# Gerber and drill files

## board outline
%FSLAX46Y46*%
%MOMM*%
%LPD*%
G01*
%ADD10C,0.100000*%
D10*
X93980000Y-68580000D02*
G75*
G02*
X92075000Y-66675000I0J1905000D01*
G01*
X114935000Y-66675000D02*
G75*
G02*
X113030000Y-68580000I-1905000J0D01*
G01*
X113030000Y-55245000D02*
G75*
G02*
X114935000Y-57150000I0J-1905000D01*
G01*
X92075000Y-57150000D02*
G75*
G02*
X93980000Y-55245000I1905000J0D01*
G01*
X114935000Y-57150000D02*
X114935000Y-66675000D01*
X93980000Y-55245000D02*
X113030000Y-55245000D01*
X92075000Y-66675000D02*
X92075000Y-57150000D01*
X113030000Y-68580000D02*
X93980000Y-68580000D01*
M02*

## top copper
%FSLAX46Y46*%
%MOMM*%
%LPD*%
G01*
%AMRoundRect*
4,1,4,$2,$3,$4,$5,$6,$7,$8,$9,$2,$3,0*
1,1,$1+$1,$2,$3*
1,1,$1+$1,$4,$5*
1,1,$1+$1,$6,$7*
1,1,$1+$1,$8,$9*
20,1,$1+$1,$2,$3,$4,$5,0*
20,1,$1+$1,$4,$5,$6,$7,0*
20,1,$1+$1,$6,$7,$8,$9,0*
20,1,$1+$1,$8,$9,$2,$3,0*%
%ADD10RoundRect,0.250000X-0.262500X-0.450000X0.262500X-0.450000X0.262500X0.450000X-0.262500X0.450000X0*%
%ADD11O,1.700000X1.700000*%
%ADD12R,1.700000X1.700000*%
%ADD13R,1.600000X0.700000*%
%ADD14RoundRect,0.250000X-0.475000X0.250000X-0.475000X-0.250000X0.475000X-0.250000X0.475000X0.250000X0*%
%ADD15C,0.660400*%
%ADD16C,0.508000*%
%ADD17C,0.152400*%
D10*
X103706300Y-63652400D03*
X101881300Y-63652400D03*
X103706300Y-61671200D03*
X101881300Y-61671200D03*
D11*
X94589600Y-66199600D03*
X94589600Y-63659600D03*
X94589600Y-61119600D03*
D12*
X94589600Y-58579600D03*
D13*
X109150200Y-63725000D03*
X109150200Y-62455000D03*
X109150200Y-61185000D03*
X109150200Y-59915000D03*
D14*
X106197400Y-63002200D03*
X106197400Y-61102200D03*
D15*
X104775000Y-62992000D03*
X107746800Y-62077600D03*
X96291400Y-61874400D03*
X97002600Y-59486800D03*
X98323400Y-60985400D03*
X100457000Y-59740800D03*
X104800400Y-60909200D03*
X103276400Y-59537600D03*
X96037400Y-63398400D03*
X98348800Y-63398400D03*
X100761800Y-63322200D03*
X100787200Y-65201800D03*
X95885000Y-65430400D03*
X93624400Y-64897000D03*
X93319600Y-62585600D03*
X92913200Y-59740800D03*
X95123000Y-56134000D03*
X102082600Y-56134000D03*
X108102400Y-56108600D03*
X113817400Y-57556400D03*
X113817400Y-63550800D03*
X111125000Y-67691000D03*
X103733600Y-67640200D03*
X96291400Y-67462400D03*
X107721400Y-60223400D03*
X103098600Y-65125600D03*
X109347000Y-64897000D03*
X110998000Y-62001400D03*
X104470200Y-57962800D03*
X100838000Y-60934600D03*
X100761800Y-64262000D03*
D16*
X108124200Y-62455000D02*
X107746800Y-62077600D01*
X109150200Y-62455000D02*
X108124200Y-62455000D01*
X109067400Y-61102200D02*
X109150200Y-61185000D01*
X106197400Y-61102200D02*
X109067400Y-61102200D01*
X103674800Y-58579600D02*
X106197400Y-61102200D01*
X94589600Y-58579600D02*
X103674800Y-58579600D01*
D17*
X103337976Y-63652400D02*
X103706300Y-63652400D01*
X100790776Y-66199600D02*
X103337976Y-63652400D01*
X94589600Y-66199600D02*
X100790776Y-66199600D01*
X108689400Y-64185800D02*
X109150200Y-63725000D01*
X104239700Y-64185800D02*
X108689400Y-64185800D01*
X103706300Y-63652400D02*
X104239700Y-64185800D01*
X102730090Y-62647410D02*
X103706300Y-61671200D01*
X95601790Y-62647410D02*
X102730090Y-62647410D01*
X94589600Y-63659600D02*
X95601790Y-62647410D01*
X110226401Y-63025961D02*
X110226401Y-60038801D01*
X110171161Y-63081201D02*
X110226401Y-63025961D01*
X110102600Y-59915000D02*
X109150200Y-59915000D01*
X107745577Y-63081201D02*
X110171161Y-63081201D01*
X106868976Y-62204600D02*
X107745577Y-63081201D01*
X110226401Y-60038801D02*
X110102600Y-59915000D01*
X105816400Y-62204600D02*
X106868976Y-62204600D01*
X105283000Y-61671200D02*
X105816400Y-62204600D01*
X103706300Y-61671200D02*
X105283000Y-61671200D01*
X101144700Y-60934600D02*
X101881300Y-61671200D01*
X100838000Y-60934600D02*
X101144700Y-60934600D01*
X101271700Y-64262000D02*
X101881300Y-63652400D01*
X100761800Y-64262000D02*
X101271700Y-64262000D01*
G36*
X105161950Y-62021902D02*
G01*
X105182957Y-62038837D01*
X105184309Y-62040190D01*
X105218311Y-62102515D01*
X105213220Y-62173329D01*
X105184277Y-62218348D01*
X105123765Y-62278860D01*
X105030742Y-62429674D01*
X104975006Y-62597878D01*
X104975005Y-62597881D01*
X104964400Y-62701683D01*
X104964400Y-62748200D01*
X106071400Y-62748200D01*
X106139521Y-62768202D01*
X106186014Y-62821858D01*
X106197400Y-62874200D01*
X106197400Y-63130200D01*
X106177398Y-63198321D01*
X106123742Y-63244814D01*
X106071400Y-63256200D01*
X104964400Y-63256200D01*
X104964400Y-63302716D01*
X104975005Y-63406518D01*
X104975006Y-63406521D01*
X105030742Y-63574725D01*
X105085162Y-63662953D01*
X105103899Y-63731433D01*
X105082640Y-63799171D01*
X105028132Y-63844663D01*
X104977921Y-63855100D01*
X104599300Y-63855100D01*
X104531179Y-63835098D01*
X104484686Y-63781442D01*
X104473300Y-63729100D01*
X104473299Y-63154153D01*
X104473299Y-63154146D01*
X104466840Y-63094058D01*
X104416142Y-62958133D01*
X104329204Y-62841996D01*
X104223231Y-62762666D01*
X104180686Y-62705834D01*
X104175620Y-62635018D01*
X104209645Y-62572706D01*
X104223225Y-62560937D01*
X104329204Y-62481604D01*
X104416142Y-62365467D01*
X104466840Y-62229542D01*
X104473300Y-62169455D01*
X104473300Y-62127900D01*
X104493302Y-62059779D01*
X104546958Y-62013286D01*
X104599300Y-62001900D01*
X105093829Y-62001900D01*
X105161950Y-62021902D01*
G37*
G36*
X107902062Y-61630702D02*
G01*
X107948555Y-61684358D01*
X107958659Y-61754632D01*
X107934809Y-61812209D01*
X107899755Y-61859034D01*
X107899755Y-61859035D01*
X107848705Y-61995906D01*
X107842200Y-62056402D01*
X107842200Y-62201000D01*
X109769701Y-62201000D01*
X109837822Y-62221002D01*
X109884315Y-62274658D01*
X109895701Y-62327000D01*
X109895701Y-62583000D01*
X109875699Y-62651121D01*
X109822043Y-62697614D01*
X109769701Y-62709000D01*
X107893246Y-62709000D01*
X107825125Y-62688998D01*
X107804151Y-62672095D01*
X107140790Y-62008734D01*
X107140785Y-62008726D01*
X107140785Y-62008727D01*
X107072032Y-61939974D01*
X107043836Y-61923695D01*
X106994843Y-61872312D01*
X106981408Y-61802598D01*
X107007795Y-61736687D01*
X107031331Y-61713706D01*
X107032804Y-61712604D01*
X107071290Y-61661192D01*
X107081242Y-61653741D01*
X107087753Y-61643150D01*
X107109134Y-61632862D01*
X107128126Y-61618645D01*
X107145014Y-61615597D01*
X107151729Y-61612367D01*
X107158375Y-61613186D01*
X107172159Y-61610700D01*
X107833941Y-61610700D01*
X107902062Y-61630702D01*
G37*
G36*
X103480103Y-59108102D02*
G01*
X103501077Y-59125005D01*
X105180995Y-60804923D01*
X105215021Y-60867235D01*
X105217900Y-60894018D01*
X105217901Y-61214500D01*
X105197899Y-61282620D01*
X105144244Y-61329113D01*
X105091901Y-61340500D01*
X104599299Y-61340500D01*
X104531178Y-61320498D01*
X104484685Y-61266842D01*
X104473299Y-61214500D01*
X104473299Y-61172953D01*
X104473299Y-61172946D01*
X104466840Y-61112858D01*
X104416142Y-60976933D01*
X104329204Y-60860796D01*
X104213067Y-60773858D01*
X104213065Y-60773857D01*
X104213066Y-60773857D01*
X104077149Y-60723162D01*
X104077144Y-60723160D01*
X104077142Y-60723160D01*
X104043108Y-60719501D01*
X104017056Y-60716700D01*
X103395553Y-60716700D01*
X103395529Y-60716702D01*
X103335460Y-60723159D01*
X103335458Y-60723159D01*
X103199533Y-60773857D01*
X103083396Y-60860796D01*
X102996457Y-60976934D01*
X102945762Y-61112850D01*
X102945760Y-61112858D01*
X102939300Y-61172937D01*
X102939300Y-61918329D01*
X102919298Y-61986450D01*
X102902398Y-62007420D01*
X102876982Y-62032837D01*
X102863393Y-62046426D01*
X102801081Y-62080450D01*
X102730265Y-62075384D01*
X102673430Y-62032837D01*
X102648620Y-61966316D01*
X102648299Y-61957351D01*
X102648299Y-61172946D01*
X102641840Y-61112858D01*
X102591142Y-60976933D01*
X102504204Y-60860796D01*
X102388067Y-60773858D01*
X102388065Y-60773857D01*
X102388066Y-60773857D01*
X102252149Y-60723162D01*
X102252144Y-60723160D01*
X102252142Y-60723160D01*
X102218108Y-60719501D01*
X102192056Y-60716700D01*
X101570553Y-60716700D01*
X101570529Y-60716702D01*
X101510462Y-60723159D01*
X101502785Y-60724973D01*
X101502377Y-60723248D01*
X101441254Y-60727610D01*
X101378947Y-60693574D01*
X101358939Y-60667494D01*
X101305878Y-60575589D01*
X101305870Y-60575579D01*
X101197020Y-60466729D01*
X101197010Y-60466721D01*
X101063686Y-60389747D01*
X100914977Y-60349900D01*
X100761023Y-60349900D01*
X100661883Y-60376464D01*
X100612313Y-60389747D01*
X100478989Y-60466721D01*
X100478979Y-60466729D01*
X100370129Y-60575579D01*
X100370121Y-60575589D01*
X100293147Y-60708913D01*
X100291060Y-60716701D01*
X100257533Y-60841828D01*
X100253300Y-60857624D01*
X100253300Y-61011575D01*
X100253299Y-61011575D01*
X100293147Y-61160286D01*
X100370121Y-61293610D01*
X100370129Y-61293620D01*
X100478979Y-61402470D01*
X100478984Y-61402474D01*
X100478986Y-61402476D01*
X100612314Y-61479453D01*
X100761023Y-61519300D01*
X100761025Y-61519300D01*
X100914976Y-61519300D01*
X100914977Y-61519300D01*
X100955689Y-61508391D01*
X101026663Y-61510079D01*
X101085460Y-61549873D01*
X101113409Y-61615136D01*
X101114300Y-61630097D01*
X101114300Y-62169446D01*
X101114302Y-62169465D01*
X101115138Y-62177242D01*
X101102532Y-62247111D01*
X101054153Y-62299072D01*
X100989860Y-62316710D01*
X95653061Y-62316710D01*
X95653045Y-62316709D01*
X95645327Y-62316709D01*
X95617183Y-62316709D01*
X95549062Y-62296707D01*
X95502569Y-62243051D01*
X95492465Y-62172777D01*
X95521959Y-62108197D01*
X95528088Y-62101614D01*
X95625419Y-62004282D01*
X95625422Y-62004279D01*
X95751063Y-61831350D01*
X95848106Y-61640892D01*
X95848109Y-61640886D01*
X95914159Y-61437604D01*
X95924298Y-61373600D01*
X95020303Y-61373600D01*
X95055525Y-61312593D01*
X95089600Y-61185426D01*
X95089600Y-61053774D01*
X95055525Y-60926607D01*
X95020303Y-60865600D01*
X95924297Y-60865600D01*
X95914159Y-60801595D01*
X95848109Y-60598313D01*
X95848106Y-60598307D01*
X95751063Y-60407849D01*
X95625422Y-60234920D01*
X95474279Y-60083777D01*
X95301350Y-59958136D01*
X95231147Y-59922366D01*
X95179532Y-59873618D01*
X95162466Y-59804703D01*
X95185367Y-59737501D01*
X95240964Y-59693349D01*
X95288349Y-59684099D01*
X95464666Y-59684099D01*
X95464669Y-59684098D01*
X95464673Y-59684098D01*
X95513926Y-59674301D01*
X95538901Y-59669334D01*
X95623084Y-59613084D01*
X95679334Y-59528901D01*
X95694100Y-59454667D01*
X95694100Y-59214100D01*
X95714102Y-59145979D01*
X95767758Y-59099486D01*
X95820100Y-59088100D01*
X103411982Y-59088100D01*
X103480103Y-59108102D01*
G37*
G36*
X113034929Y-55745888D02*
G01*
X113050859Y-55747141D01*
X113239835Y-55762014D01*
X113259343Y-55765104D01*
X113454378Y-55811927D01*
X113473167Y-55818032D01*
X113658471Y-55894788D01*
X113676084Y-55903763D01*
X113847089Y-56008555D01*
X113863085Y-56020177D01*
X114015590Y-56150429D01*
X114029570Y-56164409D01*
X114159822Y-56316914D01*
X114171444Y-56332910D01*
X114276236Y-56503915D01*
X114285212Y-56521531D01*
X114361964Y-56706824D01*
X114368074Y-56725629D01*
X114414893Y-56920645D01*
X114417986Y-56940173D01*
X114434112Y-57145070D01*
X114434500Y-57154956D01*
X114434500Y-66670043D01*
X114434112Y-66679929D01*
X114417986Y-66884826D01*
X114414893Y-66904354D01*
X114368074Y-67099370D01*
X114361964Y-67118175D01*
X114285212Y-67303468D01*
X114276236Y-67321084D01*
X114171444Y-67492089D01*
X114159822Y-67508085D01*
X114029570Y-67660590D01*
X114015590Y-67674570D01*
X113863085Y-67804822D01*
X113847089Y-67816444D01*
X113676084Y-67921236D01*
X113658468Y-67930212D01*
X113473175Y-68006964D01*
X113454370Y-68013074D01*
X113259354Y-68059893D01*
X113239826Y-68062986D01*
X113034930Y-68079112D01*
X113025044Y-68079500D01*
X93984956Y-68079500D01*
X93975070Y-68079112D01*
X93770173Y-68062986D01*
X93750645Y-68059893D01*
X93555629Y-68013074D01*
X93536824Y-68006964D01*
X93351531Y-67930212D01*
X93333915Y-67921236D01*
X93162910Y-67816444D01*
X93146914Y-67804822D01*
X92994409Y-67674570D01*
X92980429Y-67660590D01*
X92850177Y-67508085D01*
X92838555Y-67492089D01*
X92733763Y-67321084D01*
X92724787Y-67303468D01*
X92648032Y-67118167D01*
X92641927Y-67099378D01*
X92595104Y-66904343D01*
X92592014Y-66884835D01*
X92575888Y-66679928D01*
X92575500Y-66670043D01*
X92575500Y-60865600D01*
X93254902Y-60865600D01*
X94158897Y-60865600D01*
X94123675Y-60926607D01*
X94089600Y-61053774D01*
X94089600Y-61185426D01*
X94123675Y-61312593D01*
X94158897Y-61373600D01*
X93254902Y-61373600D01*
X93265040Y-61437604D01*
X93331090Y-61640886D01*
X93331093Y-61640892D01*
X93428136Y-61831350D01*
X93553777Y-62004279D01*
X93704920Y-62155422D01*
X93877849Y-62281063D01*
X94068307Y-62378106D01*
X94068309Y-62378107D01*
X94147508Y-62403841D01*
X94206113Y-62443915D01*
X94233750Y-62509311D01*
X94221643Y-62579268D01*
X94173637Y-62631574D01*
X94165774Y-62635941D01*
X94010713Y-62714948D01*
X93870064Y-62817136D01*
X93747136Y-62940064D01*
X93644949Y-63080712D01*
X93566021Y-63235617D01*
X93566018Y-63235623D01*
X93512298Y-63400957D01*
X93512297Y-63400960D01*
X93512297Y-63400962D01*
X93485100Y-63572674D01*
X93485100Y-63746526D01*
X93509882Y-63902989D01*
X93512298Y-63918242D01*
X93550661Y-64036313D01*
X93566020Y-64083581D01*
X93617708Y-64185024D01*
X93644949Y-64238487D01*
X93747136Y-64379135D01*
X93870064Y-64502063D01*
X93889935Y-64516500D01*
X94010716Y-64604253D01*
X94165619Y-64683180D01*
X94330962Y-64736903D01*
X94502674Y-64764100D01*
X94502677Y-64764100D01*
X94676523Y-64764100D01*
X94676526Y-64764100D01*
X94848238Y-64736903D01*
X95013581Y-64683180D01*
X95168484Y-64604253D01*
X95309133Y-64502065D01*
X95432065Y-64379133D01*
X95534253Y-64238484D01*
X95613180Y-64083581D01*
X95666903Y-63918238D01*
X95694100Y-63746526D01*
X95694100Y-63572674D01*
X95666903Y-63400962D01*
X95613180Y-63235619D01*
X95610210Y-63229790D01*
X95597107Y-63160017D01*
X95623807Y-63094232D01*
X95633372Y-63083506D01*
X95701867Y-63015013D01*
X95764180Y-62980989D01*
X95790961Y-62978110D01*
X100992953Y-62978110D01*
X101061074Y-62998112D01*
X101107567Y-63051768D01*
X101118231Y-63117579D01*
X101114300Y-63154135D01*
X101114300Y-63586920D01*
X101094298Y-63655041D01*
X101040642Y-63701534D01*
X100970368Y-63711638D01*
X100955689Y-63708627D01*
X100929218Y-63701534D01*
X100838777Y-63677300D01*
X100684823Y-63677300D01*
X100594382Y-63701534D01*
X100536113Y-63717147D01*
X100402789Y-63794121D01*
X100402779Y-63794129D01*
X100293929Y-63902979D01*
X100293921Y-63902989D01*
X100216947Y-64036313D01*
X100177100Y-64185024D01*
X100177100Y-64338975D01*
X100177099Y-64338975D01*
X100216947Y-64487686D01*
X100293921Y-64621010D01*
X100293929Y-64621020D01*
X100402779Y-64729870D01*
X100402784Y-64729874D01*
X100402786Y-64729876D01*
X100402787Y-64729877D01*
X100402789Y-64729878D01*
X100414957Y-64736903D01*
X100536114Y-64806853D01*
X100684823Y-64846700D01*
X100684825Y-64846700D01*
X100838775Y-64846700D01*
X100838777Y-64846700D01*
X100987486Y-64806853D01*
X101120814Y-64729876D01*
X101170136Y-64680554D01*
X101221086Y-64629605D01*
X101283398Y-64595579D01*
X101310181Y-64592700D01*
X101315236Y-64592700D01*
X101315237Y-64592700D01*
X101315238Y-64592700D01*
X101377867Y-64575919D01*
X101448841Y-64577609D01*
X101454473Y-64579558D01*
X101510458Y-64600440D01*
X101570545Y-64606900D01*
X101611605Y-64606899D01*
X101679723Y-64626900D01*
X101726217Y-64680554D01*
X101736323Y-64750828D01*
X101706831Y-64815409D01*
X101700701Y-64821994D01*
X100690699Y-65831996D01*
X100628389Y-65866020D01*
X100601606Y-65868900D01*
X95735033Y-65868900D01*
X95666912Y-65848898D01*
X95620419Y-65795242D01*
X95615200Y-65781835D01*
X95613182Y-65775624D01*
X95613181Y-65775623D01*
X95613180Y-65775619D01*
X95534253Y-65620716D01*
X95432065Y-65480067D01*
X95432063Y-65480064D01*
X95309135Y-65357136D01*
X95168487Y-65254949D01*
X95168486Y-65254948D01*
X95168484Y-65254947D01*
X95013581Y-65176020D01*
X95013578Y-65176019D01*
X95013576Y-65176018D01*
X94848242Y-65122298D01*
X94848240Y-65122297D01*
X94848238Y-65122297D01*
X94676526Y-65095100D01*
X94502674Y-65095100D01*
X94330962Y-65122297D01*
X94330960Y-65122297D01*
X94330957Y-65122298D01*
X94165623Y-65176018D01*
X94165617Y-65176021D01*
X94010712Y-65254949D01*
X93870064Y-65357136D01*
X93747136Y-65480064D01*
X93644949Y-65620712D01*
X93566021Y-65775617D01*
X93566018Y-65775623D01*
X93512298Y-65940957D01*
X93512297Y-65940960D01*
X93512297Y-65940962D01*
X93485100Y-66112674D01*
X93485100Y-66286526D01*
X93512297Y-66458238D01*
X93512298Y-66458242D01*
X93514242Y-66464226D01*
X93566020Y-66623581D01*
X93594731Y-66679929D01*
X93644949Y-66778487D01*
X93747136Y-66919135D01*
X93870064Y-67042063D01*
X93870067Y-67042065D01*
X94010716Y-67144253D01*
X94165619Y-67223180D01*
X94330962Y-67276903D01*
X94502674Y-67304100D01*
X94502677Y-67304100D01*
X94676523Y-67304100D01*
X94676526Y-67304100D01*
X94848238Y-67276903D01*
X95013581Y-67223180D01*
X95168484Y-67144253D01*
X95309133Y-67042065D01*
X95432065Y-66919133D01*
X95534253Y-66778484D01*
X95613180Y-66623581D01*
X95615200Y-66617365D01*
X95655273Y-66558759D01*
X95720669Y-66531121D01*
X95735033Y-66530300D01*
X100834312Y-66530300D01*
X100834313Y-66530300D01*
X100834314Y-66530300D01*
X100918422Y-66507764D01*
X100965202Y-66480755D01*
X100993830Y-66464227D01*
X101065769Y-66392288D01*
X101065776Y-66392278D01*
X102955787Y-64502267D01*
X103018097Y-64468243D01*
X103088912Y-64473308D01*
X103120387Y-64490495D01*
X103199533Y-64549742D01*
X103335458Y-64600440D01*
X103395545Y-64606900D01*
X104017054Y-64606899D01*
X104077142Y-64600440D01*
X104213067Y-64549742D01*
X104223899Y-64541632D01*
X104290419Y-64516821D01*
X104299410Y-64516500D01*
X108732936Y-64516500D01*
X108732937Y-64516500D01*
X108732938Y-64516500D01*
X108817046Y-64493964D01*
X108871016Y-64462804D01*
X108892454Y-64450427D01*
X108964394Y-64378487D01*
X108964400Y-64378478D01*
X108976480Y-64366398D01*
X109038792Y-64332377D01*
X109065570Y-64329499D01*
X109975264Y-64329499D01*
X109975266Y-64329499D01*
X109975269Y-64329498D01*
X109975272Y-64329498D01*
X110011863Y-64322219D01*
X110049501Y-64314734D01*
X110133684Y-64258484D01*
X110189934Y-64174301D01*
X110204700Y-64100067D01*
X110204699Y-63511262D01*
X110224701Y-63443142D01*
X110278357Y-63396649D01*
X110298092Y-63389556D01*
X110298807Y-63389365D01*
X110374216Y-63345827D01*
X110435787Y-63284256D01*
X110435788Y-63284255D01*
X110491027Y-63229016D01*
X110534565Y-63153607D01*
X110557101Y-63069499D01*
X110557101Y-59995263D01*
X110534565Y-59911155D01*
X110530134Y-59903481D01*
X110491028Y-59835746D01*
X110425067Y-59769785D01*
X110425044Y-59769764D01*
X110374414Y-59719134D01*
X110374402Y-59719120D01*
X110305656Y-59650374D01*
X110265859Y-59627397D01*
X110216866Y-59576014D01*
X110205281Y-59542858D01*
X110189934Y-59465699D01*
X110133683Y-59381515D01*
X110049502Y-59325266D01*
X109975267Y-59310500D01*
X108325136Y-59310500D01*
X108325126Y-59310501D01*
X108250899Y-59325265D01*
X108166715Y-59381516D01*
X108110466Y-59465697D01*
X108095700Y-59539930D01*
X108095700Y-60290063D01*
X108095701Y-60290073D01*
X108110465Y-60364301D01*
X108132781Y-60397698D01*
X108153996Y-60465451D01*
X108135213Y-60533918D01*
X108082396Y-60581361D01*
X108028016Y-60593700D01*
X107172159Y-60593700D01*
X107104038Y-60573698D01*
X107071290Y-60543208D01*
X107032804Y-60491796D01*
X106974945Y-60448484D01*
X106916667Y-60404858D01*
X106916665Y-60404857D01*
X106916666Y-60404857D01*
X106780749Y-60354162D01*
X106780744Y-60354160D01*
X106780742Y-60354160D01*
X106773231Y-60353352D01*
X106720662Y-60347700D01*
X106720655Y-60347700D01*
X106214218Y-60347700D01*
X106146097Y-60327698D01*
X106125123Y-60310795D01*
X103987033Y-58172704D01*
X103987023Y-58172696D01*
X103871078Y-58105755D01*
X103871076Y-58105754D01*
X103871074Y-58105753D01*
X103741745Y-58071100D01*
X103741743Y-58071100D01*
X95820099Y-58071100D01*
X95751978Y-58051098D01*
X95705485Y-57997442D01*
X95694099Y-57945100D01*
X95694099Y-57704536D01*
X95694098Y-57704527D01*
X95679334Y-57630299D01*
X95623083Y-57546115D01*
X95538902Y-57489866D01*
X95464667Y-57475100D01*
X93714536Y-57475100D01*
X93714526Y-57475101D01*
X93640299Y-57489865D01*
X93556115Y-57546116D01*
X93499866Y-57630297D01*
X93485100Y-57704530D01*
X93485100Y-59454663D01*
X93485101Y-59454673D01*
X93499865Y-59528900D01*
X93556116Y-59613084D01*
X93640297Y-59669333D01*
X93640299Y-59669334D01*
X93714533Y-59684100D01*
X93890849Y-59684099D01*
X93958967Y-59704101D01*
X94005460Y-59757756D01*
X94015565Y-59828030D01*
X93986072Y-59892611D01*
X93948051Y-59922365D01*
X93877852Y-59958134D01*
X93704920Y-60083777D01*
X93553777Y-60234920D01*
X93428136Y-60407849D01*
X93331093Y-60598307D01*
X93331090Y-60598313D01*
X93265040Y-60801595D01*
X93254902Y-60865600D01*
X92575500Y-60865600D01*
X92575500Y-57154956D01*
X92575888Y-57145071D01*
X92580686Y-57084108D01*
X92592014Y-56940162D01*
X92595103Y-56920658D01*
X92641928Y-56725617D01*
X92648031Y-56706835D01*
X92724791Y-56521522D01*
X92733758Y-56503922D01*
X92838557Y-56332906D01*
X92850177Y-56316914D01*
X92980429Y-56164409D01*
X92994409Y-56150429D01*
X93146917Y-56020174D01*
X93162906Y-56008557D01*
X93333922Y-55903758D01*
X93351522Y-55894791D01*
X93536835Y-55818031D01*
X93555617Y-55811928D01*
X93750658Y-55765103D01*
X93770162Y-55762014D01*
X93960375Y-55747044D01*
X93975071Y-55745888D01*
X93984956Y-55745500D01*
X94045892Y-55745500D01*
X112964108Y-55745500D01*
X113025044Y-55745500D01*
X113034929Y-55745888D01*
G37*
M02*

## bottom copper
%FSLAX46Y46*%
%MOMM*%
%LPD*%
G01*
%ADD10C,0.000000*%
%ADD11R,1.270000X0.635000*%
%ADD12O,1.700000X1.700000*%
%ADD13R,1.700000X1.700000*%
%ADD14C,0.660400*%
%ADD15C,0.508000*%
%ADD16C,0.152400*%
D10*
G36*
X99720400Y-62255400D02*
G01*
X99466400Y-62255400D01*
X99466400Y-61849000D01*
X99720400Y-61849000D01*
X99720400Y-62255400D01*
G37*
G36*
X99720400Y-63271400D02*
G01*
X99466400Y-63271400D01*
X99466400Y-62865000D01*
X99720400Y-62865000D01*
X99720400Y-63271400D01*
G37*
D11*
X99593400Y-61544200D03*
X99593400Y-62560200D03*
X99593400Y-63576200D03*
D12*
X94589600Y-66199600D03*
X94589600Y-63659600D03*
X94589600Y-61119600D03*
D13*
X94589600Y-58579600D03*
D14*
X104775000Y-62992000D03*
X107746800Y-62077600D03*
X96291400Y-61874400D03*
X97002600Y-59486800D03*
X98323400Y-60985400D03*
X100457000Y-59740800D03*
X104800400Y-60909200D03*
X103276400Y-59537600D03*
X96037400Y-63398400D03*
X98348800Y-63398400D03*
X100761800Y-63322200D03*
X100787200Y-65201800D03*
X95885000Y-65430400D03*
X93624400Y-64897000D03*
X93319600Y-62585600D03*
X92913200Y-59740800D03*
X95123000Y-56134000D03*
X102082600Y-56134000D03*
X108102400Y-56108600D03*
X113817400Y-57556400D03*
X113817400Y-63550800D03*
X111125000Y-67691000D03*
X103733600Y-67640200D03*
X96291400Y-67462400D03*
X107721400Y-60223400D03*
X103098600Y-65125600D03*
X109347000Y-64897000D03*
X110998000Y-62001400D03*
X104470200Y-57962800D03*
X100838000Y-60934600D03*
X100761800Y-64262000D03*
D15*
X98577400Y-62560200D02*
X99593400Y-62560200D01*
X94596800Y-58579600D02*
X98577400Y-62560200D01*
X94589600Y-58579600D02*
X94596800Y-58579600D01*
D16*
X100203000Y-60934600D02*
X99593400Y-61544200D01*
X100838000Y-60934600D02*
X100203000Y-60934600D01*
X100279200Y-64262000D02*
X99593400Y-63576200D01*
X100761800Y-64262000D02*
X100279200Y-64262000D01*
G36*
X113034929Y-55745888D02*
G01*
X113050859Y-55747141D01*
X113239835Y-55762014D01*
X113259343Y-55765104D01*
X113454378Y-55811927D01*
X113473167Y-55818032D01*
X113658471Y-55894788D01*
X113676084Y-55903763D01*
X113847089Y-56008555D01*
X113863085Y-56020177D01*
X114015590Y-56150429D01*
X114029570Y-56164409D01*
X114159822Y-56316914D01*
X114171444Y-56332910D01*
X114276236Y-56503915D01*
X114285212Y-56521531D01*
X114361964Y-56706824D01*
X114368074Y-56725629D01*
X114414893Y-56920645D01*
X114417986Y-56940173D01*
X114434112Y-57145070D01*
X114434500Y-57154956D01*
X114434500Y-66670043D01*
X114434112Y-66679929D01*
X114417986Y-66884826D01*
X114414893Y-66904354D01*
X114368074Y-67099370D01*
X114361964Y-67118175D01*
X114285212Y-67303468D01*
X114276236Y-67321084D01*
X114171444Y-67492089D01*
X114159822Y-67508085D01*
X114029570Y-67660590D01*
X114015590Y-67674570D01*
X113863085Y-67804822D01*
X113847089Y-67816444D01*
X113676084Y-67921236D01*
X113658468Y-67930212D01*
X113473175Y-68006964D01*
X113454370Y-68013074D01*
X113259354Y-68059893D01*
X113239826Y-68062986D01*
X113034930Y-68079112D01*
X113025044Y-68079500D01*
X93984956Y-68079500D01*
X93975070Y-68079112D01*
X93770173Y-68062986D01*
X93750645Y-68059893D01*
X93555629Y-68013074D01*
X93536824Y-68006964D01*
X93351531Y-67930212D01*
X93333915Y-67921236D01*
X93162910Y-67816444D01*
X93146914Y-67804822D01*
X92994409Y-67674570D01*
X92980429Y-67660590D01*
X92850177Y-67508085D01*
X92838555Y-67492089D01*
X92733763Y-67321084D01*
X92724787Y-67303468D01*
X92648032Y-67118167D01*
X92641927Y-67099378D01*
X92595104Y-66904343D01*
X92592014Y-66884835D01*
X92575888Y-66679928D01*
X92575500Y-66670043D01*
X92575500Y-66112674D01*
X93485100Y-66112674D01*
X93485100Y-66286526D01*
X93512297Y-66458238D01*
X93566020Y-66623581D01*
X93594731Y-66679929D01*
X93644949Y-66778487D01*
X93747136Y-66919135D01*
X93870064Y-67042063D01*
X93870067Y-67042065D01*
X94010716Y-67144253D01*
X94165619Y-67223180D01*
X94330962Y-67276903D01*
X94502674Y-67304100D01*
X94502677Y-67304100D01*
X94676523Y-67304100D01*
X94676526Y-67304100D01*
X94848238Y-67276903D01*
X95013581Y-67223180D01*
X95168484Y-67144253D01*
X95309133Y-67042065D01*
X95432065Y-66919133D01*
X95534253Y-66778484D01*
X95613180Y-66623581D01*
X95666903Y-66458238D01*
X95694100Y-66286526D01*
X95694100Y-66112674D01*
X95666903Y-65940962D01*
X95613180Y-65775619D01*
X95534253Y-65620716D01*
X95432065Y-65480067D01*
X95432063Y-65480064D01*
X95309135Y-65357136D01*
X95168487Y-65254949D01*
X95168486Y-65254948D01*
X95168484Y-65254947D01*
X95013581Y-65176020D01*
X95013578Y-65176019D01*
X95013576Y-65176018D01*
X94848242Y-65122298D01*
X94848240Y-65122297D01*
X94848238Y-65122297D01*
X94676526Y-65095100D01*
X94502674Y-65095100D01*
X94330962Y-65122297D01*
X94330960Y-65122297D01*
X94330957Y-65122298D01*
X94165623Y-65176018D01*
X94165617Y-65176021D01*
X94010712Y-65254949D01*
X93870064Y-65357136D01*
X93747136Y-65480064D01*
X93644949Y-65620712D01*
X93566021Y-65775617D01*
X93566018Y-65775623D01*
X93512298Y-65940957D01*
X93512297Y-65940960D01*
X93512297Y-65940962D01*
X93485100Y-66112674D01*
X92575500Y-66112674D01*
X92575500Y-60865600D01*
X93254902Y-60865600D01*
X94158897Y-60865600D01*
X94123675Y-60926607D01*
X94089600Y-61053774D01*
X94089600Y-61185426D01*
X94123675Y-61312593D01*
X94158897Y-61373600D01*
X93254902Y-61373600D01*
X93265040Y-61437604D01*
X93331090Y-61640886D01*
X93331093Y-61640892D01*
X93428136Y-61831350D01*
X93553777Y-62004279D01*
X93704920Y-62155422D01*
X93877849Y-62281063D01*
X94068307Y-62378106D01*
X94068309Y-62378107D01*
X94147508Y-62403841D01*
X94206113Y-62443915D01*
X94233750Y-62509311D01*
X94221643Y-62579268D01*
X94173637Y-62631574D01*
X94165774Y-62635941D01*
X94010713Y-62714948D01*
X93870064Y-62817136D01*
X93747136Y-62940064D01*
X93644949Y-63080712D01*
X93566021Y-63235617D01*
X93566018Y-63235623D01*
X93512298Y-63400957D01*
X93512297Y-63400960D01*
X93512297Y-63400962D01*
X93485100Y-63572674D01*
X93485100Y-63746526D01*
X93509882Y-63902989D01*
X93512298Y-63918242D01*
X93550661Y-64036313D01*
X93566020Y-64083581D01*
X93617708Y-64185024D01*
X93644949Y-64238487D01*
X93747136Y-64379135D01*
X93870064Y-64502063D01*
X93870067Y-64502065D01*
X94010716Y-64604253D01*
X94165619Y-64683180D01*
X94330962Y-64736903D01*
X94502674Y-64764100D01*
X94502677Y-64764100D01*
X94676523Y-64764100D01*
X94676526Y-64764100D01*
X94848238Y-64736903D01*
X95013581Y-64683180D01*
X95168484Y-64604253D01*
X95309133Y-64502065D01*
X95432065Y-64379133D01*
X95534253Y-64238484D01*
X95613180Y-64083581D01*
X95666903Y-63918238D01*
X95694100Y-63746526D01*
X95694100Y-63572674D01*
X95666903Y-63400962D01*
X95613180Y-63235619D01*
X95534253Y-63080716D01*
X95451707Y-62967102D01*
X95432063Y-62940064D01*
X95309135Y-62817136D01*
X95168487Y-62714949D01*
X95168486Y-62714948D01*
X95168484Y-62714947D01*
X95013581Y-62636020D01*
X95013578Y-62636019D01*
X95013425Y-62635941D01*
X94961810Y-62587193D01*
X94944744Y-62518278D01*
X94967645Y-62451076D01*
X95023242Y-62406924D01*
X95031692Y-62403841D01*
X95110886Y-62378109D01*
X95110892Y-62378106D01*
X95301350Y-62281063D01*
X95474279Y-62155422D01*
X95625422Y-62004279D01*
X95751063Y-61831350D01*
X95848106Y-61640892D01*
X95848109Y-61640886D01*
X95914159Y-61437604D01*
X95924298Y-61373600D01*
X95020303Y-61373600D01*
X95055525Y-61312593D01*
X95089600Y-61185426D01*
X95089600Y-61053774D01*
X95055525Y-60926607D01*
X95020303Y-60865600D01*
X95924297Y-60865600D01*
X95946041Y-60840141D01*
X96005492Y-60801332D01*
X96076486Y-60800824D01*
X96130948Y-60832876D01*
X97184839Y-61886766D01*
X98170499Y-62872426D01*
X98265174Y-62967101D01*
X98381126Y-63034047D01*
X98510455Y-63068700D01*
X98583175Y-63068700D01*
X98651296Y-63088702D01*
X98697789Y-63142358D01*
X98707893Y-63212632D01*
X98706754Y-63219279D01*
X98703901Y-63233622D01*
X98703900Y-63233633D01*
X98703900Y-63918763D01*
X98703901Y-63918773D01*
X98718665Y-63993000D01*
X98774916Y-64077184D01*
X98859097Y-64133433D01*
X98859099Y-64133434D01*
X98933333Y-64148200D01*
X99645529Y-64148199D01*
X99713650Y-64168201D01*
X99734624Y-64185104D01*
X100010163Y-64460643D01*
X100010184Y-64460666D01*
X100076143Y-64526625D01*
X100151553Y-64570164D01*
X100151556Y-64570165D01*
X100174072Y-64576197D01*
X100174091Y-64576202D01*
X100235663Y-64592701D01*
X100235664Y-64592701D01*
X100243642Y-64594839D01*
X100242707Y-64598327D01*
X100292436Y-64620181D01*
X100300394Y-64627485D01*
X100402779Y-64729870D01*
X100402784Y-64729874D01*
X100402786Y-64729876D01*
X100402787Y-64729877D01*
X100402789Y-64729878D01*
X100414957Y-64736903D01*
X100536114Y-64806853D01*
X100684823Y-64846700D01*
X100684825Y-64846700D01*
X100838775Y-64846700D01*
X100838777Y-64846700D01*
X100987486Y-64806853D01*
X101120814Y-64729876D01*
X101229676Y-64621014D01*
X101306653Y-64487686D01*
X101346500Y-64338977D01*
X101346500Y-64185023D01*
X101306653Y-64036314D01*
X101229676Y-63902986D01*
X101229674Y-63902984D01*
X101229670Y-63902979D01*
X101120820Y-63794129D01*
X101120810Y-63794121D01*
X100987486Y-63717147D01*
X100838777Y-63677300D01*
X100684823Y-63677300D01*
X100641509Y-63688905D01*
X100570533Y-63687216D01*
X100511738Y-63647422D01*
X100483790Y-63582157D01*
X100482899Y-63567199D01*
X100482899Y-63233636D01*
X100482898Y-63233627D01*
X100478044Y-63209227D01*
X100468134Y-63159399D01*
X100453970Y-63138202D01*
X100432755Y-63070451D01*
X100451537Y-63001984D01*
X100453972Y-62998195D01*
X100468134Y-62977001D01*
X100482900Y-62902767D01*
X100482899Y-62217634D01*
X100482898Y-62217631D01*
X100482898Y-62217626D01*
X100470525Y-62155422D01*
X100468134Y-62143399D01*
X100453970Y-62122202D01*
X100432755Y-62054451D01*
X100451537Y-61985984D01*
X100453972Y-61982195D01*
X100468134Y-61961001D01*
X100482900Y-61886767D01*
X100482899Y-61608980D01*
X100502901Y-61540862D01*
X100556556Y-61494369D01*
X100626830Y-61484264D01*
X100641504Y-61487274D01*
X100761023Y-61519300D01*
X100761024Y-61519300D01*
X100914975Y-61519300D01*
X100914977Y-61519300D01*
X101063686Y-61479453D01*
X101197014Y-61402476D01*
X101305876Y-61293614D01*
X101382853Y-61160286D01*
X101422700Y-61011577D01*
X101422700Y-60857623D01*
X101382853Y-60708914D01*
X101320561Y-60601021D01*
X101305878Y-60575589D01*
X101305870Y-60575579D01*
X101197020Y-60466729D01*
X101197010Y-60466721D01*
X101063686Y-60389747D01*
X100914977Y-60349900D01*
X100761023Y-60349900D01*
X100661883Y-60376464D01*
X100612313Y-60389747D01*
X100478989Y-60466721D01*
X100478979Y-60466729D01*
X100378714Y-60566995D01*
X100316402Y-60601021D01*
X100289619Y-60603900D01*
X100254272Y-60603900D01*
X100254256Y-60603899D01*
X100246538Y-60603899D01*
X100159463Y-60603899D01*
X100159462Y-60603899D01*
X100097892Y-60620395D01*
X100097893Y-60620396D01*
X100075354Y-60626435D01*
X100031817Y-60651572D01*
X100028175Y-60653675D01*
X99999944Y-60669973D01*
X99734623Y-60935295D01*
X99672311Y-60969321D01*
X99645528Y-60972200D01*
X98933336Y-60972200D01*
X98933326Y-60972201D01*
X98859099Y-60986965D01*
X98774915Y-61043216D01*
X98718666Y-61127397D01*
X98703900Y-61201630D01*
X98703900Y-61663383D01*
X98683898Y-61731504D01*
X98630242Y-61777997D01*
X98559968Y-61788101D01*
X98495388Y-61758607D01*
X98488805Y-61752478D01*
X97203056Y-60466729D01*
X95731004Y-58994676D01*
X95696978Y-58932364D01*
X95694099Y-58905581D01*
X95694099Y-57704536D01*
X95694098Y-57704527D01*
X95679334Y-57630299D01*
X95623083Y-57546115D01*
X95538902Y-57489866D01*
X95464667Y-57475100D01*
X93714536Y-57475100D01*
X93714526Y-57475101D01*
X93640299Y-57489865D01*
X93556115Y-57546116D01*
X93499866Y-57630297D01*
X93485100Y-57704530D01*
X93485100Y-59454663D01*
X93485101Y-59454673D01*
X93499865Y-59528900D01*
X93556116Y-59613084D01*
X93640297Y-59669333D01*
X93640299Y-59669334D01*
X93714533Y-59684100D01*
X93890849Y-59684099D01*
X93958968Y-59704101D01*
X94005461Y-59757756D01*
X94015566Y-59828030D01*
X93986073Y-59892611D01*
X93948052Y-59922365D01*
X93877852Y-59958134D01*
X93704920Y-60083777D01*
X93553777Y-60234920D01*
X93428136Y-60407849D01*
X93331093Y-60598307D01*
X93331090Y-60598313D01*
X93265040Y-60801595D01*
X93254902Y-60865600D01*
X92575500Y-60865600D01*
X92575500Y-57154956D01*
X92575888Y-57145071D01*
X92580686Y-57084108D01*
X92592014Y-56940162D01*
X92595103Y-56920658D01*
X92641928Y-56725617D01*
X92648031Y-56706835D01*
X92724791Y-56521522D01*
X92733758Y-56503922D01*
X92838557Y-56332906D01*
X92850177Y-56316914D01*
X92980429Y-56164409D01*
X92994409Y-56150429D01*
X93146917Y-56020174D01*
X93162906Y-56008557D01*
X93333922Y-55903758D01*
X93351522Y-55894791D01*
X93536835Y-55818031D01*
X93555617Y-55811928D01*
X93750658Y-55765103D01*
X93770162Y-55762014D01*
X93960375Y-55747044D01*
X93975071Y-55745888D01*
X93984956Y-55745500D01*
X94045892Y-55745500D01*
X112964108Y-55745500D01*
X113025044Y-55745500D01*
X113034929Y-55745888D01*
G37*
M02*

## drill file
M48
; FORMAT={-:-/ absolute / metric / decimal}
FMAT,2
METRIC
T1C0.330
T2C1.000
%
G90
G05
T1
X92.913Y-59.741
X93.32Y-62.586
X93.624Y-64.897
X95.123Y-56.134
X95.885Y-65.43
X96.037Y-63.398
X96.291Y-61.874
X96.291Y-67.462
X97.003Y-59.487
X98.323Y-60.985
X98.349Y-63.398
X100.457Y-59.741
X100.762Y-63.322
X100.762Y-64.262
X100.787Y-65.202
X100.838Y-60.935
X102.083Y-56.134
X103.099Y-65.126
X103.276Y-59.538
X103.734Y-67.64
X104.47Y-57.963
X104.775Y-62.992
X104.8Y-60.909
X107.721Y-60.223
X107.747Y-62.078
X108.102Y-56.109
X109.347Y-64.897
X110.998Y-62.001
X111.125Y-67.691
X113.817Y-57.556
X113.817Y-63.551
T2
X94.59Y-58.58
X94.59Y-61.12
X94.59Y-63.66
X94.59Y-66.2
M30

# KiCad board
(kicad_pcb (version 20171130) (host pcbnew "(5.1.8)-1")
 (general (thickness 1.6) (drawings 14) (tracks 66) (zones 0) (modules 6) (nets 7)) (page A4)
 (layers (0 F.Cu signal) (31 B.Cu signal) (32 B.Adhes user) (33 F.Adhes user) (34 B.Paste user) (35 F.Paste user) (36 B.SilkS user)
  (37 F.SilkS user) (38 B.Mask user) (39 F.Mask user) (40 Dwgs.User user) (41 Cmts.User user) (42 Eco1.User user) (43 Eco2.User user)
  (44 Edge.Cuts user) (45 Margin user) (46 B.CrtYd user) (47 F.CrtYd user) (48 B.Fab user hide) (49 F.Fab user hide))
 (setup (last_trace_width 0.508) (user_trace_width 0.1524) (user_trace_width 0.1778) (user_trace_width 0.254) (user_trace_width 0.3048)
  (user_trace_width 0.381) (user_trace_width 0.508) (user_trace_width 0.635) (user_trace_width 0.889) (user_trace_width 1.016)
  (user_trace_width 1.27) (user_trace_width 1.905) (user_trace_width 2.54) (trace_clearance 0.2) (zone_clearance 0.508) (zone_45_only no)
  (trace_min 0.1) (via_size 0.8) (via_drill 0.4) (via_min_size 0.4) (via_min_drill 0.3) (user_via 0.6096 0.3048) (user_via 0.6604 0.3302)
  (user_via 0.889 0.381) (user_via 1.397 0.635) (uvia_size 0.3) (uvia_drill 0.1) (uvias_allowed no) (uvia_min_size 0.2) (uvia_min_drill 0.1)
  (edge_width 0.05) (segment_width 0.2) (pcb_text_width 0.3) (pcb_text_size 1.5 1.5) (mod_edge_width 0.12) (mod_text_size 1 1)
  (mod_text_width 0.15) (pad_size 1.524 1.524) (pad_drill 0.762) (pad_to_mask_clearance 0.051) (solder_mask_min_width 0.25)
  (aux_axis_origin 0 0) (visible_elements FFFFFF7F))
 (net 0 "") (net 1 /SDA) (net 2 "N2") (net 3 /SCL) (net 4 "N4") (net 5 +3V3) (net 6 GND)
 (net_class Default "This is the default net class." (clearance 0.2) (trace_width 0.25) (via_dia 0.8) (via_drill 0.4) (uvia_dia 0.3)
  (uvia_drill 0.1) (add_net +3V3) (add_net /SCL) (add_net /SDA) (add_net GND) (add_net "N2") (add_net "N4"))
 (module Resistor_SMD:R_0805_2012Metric (layer F.Cu) (at 102.7938 63.6524)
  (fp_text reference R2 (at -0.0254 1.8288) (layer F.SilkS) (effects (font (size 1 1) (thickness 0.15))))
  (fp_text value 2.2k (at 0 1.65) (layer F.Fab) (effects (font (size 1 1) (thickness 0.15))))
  (pad 2 smd roundrect (at 0.9125 0) (size 1.025 1.4) (layers F.Cu F.Paste F.Mask) (roundrect_rratio 0.243902) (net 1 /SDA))
  (pad 1 smd roundrect (at -0.9125 0) (size 1.025 1.4) (layers F.Cu F.Paste F.Mask) (roundrect_rratio 0.243902) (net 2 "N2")))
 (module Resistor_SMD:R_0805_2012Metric (layer F.Cu) (at 102.7938 61.6712)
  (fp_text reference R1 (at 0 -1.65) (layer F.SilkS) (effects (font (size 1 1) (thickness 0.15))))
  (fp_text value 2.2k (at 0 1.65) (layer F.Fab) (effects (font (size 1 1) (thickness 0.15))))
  (pad 2 smd roundrect (at 0.9125 0) (size 1.025 1.4) (layers F.Cu F.Paste F.Mask) (roundrect_rratio 0.243902) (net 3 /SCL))
  (pad 1 smd roundrect (at -0.9125 0) (size 1.025 1.4) (layers F.Cu F.Paste F.Mask) (roundrect_rratio 0.243902) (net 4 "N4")))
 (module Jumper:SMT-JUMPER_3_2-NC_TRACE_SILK (layer B.Cu) (at 99.5934 62.5602 90)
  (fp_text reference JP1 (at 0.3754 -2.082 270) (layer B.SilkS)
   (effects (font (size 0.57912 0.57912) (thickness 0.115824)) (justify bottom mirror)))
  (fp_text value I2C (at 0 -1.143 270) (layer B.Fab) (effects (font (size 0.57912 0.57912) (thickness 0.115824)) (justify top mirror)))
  (fp_poly (pts (xy 0.3048 -0.127) (xy 0.7112 -0.127) (xy 0.7112 0.127) (xy 0.3048 0.127)) (layer B.Cu) (width 0))
  (fp_poly (pts (xy -0.7112 -0.127) (xy -0.3048 -0.127) (xy -0.3048 0.127) (xy -0.7112 0.127)) (layer B.Cu) (width 0))
  (pad 3 smd rect (at 1.016 0 90) (size 0.635 1.27) (layers B.Cu B.Mask) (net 4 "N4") (solder_mask_margin 0.1016))
  (pad 2 smd rect (at 0 0 90) (size 0.635 1.27) (layers B.Cu B.Mask) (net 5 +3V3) (solder_mask_margin 0.1016))
  (pad 1 smd rect (at -1.016 0 90) (size 0.635 1.27) (layers B.Cu B.Mask) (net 2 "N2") (solder_mask_margin 0.1016)))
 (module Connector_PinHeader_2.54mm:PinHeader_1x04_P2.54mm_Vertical (layer F.Cu) (at 94.5896 58.5796)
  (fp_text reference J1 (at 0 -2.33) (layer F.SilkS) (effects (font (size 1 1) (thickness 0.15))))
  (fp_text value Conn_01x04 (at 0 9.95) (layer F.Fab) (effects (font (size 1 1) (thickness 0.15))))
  (pad 4 thru_hole oval (at 0 7.62) (size 1.7 1.7) (drill 1) (layers *.Cu *.Mask) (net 1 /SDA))
  (pad 3 thru_hole oval (at 0 5.08) (size 1.7 1.7) (drill 1) (layers *.Cu *.Mask) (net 3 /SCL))
  (pad 2 thru_hole oval (at 0 2.54) (size 1.7 1.7) (drill 1) (layers *.Cu *.Mask) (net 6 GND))
  (pad 1 thru_hole rect (at 0 0) (size 1.7 1.7) (drill 1) (layers *.Cu *.Mask) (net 5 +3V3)))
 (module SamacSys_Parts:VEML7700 (layer F.Cu) (at 109.5502 58.42 270)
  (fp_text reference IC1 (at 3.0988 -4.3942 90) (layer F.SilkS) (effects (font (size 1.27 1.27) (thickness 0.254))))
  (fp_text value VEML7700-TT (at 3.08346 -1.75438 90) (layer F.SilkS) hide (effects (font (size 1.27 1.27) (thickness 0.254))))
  (pad 4 smd rect (at 5.305 0.4 270) (size 0.7 1.6) (layers F.Cu F.Paste F.Mask) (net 1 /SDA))
  (pad 3 smd rect (at 4.035 0.4 270) (size 0.7 1.6) (layers F.Cu F.Paste F.Mask) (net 6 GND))
  (pad 2 smd rect (at 2.765 0.4 270) (size 0.7 1.6) (layers F.Cu F.Paste F.Mask) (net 5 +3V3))
  (pad 1 smd rect (at 1.495 0.4 270) (size 0.7 1.6) (layers F.Cu F.Paste F.Mask) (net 3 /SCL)))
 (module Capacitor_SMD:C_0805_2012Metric (layer F.Cu) (at 106.1974 62.0522 270)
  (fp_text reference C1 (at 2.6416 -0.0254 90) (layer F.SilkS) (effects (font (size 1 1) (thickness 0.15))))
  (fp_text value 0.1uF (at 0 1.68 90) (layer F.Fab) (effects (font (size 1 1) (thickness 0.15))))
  (pad 2 smd roundrect (at 0.95 0 270) (size 1 1.45) (layers F.Cu F.Paste F.Mask) (roundrect_rratio 0.25) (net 6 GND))
  (pad 1 smd roundrect (at -0.95 0 270) (size 1 1.45) (layers F.Cu F.Paste F.Mask) (roundrect_rratio 0.25) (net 5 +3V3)))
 (gr_arc (start 93.98 66.675) (end 92.075 66.675) (angle -90) (layer Edge.Cuts) (width 0.1))
 (gr_arc (start 113.03 66.675) (end 113.03 68.58) (angle -90) (layer Edge.Cuts) (width 0.1))
 (gr_arc (start 113.03 57.15) (end 114.935 57.15) (angle -90) (layer Edge.Cuts) (width 0.1))
 (gr_arc (start 93.98 57.15) (end 93.98 55.245) (angle -90) (layer Edge.Cuts) (width 0.1))
 (gr_line (start 114.935 57.15) (end 114.935 66.675) (layer Edge.Cuts) (width 0.1))
 (gr_line (start 93.98 55.245) (end 113.03 55.245) (layer Edge.Cuts) (width 0.1))
 (gr_line (start 92.075 66.675) (end 92.075 57.15) (layer Edge.Cuts) (width 0.1))
 (gr_line (start 113.03 68.58) (end 93.98 68.58) (layer Edge.Cuts) (width 0.1))
 (via (at 104.775 62.992) (size 0.6604) (drill 0.3302) (layers F.Cu B.Cu) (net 6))
 (via (at 107.7468 62.0776) (size 0.6604) (drill 0.3302) (layers F.Cu B.Cu) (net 6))
 (segment (start 108.1242 62.455) (end 107.7468 62.0776) (width 0.508) (layer F.Cu) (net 6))
 (segment (start 109.1502 62.455) (end 108.1242 62.455) (width 0.508) (layer F.Cu) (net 6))
 (via (at 96.2914 61.8744) (size 0.6604) (drill 0.3302) (layers F.Cu B.Cu) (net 6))
 (via (at 97.0026 59.4868) (size 0.6604) (drill 0.3302) (layers F.Cu B.Cu) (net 6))
 (via (at 98.3234 60.9854) (size 0.6604) (drill 0.3302) (layers F.Cu B.Cu) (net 6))
 (via (at 100.457 59.7408) (size 0.6604) (drill 0.3302) (layers F.Cu B.Cu) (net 6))
 (via (at 104.8004 60.9092) (size 0.6604) (drill 0.3302) (layers F.Cu B.Cu) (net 6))
 (via (at 103.2764 59.5376) (size 0.6604) (drill 0.3302) (layers F.Cu B.Cu) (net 6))
 (via (at 96.0374 63.3984) (size 0.6604) (drill 0.3302) (layers F.Cu B.Cu) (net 6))
 (via (at 98.3488 63.3984) (size 0.6604) (drill 0.3302) (layers F.Cu B.Cu) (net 6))
 (via (at 100.7618 63.3222) (size 0.6604) (drill 0.3302) (layers F.Cu B.Cu) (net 6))
 (via (at 100.7872 65.2018) (size 0.6604) (drill 0.3302) (layers F.Cu B.Cu) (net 6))
 (via (at 95.885 65.4304) (size 0.6604) (drill 0.3302) (layers F.Cu B.Cu) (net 6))
 (via (at 93.6244 64.897) (size 0.6604) (drill 0.3302) (layers F.Cu B.Cu) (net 6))
 (via (at 93.3196 62.5856) (size 0.6604) (drill 0.3302) (layers F.Cu B.Cu) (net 6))
 (via (at 92.9132 59.7408) (size 0.6604) (drill 0.3302) (layers F.Cu B.Cu) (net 6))
 (via (at 95.123 56.134) (size 0.6604) (drill 0.3302) (layers F.Cu B.Cu) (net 6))
 (via (at 102.0826 56.134) (size 0.6604) (drill 0.3302) (layers F.Cu B.Cu) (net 6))
 (via (at 108.1024 56.1086) (size 0.6604) (drill 0.3302) (layers F.Cu B.Cu) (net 6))
 (via (at 113.8174 57.5564) (size 0.6604) (drill 0.3302) (layers F.Cu B.Cu) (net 6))
 (via (at 113.8174 63.5508) (size 0.6604) (drill 0.3302) (layers F.Cu B.Cu) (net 6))
 (via (at 111.125 67.691) (size 0.6604) (drill 0.3302) (layers F.Cu B.Cu) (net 6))
 (via (at 103.7336 67.6402) (size 0.6604) (drill 0.3302) (layers F.Cu B.Cu) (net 6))
 (via (at 96.2914 67.4624) (size 0.6604) (drill 0.3302) (layers F.Cu B.Cu) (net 6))
 (via (at 107.7214 60.2234) (size 0.6604) (drill 0.3302) (layers F.Cu B.Cu) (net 6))
 (via (at 103.0986 65.1256) (size 0.6604) (drill 0.3302) (layers F.Cu B.Cu) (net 6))
 (via (at 109.347 64.897) (size 0.6604) (drill 0.3302) (layers F.Cu B.Cu) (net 6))
 (via (at 110.998 62.0014) (size 0.6604) (drill 0.3302) (layers F.Cu B.Cu) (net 6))
 (via (at 104.4702 57.9628) (size 0.6604) (drill 0.3302) (layers F.Cu B.Cu) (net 6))
 (segment (start 109.0674 61.1022) (end 109.1502 61.185) (width 0.508) (layer F.Cu) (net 5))
 (segment (start 106.1974 61.1022) (end 109.0674 61.1022) (width 0.508) (layer F.Cu) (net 5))
 (segment (start 98.5774 62.5602) (end 99.5934 62.5602) (width 0.508) (layer B.Cu) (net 5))
 (segment (start 94.5968 58.5796) (end 98.5774 62.5602) (width 0.508) (layer B.Cu) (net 5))
 (segment (start 94.5896 58.5796) (end 94.5968 58.5796) (width 0.508) (layer B.Cu) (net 5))
 (segment (start 103.6748 58.5796) (end 106.1974 61.1022) (width 0.508) (layer F.Cu) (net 5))
 (segment (start 94.5896 58.5796) (end 103.6748 58.5796) (width 0.508) (layer F.Cu) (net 5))
 (segment (start 103.337976 63.6524) (end 103.7063 63.6524) (width 0.1524) (layer F.Cu) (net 1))
 (segment (start 100.790776 66.1996) (end 103.337976 63.6524) (width 0.1524) (layer F.Cu) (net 1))
 (segment (start 94.5896 66.1996) (end 100.790776 66.1996) (width 0.1524) (layer F.Cu) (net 1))
 (segment (start 108.6894 64.1858) (end 109.1502 63.725) (width 0.1524) (layer F.Cu) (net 1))
 (segment (start 104.2397 64.1858) (end 108.6894 64.1858) (width 0.1524) (layer F.Cu) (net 1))
 (segment (start 103.7063 63.6524) (end 104.2397 64.1858) (width 0.1524) (layer F.Cu) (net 1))
 (segment (start 102.73009 62.64741) (end 103.7063 61.6712) (width 0.1524) (layer F.Cu) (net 3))
 (segment (start 95.60179 62.64741) (end 102.73009 62.64741) (width 0.1524) (layer F.Cu) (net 3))
 (segment (start 94.5896 63.6596) (end 95.60179 62.64741) (width 0.1524) (layer F.Cu) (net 3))
 (segment (start 110.226401 63.025961) (end 110.226401 60.038801) (width 0.1524) (layer F.Cu) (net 3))
 (segment (start 110.171161 63.081201) (end 110.226401 63.025961) (width 0.1524) (layer F.Cu) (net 3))
 (segment (start 110.1026 59.915) (end 109.1502 59.915) (width 0.1524) (layer F.Cu) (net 3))
 (segment (start 107.745577 63.081201) (end 110.171161 63.081201) (width 0.1524) (layer F.Cu) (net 3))
 (segment (start 106.868976 62.2046) (end 107.745577 63.081201) (width 0.1524) (layer F.Cu) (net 3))
 (segment (start 110.226401 60.038801) (end 110.1026 59.915) (width 0.1524) (layer F.Cu) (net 3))
 (segment (start 105.8164 62.2046) (end 106.868976 62.2046) (width 0.1524) (layer F.Cu) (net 3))
 (segment (start 105.283 61.6712) (end 105.8164 62.2046) (width 0.1524) (layer F.Cu) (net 3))
 (segment (start 103.7063 61.6712) (end 105.283 61.6712) (width 0.1524) (layer F.Cu) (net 3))
 (via (at 100.838 60.9346) (size 0.6604) (drill 0.3302) (layers F.Cu B.Cu) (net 4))
 (segment (start 100.203 60.9346) (end 99.5934 61.5442) (width 0.1524) (layer B.Cu) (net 4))
 (segment (start 100.838 60.9346) (end 100.203 60.9346) (width 0.1524) (layer B.Cu) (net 4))
 (segment (start 101.1447 60.9346) (end 101.8813 61.6712) (width 0.1524) (layer F.Cu) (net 4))
 (segment (start 100.838 60.9346) (end 101.1447 60.9346) (width 0.1524) (layer F.Cu) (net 4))
 (via (at 100.7618 64.262) (size 0.6604) (drill 0.3302) (layers F.Cu B.Cu) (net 2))
 (segment (start 100.2792 64.262) (end 99.5934 63.5762) (width 0.1524) (layer B.Cu) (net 2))
 (segment (start 100.7618 64.262) (end 100.2792 64.262) (width 0.1524) (layer B.Cu) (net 2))
 (segment (start 101.2717 64.262) (end 101.8813 63.6524) (width 0.1524) (layer F.Cu) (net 2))
 (segment (start 100.7618 64.262) (end 101.2717 64.262) (width 0.1524) (layer F.Cu) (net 2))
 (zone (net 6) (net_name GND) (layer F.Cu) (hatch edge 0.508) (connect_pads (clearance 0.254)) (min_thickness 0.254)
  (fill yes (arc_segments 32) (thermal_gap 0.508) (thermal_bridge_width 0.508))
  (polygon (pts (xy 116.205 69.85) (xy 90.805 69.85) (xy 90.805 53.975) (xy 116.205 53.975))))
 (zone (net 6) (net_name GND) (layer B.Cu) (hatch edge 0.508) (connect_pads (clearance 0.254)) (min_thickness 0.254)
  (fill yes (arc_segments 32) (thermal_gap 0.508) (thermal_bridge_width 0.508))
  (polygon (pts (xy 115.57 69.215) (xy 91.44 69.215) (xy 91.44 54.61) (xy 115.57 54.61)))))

